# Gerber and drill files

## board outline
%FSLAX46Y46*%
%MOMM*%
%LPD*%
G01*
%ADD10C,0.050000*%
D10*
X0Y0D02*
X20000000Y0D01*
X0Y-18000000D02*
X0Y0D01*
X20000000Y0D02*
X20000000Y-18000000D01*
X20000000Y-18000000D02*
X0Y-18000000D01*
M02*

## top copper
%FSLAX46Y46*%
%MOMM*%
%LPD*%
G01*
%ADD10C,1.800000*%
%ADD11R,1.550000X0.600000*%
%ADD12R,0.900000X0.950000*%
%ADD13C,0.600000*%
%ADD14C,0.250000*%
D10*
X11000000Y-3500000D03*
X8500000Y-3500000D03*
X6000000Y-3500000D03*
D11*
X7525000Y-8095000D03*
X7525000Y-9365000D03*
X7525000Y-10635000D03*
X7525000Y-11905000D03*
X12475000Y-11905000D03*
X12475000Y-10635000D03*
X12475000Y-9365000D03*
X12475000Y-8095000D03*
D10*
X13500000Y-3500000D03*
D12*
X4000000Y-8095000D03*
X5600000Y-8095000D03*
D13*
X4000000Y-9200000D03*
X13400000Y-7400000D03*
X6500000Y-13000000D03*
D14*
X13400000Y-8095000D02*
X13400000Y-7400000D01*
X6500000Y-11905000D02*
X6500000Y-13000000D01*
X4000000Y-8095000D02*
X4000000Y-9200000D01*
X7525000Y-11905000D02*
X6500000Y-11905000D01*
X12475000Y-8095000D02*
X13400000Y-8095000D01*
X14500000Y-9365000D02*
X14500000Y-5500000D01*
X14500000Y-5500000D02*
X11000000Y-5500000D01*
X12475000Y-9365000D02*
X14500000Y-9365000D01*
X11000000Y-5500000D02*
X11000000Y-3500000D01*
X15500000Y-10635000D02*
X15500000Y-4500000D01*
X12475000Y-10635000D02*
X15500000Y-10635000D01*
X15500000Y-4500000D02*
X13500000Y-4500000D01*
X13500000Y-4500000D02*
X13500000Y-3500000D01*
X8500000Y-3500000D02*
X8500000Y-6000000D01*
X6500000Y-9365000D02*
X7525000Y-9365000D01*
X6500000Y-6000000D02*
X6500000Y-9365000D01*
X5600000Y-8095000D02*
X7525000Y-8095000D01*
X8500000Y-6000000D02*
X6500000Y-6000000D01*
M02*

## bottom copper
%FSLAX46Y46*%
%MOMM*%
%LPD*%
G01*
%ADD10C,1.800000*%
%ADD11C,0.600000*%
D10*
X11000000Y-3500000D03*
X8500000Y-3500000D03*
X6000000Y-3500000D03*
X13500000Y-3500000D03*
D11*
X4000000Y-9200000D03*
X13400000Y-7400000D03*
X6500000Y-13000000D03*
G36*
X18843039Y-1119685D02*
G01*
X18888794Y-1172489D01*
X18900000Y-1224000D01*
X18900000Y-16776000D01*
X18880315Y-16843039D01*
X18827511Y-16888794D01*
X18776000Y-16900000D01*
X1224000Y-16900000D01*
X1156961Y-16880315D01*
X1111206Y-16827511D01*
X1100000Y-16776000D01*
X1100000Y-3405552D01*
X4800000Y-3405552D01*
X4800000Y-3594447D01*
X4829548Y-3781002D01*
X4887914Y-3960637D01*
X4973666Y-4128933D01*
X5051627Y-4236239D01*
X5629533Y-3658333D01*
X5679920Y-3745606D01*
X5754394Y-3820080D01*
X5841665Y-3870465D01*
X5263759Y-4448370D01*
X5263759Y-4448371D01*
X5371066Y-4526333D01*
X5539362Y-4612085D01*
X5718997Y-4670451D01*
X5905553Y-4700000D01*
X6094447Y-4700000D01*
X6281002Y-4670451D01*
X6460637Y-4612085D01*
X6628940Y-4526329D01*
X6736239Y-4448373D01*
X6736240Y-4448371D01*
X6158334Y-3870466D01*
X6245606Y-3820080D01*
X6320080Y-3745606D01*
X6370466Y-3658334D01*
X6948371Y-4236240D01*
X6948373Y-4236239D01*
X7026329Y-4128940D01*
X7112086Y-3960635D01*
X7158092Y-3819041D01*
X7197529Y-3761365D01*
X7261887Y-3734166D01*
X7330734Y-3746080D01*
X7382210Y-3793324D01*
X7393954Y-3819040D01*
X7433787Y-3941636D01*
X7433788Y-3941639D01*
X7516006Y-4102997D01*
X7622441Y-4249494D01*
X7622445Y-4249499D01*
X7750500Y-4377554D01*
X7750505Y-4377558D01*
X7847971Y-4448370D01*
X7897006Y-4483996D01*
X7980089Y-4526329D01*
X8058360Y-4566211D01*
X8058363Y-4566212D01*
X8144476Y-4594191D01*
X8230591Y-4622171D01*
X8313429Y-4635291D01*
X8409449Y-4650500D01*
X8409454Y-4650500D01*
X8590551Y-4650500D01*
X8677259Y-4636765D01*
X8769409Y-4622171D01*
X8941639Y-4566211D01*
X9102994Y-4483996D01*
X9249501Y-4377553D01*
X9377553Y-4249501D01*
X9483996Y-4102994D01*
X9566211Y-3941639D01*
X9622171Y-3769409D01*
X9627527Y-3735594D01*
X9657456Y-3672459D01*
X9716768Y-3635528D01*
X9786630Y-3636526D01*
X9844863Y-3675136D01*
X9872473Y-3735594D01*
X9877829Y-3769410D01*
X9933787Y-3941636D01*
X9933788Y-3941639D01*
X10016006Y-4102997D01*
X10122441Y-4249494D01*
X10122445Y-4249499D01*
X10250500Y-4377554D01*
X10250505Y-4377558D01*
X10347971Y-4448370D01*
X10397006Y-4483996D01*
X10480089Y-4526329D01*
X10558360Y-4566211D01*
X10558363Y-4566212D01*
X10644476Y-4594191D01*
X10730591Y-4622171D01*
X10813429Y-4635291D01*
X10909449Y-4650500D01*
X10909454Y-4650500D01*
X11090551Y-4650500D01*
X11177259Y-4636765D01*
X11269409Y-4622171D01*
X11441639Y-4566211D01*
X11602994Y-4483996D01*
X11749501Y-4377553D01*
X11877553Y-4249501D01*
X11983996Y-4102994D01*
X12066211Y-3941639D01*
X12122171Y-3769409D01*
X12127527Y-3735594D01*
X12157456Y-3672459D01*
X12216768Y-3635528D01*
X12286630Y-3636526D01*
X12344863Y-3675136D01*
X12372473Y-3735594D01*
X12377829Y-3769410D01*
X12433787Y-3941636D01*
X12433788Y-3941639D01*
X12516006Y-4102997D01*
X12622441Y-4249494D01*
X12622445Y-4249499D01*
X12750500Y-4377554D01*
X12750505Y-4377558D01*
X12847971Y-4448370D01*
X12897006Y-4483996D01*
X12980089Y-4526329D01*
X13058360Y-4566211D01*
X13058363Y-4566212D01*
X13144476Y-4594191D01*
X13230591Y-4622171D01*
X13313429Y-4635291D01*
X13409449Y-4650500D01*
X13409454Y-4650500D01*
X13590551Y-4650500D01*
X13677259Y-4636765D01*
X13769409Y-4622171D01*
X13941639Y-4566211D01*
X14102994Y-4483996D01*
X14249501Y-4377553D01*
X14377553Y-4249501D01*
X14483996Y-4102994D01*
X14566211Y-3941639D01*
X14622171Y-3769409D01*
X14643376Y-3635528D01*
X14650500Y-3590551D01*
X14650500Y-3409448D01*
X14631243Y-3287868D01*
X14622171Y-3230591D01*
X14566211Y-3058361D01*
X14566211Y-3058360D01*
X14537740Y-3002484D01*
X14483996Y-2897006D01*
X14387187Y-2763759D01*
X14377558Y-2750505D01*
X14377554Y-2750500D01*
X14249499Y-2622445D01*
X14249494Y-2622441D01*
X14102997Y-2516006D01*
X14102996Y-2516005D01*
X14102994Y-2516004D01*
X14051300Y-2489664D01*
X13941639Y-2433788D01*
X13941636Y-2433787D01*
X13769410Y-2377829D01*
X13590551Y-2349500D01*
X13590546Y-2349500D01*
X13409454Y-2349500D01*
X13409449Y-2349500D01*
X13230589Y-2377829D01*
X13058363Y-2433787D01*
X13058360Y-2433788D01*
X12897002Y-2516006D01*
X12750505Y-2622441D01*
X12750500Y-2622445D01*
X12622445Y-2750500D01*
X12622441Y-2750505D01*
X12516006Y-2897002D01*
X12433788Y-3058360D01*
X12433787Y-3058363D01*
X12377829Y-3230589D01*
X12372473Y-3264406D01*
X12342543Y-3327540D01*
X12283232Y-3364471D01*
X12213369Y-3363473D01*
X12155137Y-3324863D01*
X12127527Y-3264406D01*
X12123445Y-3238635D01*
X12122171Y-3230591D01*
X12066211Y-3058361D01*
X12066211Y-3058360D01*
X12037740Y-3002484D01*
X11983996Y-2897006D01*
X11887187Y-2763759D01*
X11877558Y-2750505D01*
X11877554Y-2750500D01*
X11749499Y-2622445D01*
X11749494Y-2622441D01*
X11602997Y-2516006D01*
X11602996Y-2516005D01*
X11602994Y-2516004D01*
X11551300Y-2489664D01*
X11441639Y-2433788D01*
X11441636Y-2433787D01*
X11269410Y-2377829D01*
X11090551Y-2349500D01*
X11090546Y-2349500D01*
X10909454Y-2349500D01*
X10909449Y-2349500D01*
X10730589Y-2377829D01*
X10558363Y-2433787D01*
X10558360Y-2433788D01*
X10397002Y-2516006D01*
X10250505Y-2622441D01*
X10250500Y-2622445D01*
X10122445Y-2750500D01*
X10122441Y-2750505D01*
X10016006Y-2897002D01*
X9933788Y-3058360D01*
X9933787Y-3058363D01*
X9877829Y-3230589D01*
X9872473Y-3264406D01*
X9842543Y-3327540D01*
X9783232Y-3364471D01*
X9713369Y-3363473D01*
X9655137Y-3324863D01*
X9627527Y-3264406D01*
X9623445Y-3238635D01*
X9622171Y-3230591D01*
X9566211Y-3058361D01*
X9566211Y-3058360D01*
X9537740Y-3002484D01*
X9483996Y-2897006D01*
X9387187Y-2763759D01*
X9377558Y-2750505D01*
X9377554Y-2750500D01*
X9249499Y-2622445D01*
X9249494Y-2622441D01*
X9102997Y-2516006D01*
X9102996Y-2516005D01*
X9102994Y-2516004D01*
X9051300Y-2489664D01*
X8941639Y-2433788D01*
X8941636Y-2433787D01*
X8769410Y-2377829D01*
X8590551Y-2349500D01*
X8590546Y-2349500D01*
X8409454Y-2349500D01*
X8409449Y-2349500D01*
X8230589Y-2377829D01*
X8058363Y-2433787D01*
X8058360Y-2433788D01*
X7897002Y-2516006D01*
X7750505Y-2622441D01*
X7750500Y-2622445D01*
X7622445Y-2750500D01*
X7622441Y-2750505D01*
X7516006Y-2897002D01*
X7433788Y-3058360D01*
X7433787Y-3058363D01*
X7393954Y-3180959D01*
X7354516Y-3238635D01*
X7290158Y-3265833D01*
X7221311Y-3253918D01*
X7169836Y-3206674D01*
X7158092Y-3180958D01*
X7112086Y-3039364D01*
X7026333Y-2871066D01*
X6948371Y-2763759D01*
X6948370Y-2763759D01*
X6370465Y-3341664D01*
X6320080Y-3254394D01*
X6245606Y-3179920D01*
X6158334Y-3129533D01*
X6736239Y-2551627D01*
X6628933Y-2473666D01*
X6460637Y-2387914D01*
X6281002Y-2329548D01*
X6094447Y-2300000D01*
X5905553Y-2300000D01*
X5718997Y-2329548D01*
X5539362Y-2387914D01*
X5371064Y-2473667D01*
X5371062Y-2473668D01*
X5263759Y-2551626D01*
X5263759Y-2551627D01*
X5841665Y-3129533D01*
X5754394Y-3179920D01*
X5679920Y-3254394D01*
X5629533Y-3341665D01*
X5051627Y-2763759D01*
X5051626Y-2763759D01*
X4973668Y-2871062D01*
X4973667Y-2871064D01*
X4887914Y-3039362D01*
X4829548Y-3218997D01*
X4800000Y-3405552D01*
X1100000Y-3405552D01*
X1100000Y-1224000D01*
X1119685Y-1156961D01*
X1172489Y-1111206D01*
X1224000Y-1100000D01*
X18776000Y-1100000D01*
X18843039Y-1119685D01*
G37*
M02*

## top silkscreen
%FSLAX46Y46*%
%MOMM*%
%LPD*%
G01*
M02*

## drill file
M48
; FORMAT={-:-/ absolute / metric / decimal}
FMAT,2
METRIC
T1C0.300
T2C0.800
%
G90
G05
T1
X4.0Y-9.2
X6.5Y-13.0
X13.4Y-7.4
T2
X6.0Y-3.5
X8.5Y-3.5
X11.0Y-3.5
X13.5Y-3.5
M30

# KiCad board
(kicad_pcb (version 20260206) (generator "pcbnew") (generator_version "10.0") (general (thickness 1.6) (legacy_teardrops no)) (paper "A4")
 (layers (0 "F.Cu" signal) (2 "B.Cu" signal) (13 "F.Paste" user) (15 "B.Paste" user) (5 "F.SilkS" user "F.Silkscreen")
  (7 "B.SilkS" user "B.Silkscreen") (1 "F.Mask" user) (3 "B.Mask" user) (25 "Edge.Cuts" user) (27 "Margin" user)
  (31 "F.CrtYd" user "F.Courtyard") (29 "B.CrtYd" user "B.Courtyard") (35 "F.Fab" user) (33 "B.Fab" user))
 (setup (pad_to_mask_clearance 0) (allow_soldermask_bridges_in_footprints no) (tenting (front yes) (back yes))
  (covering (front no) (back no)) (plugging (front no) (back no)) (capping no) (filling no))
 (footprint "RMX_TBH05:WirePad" (layer "F.Cu") (at 11 3.5)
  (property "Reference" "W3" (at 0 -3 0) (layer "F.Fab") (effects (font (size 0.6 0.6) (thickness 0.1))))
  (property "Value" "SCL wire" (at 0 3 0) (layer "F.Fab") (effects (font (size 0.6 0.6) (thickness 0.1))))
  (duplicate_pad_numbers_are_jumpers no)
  (pad "1" thru_hole circle (at 0 0) (size 1.8 1.8) (drill 0.8) (layers "*.Cu" "*.Mask") (remove_unused_layers no) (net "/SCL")))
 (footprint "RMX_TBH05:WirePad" (layer "F.Cu") (at 8.5 3.5)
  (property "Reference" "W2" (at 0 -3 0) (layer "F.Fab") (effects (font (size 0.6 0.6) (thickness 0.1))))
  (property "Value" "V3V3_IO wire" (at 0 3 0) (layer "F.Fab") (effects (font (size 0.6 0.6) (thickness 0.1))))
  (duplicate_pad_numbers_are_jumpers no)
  (pad "1" thru_hole circle (at 0 0) (size 1.8 1.8) (drill 0.8) (layers "*.Cu" "*.Mask") (remove_unused_layers no) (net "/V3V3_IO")))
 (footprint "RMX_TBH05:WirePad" (layer "F.Cu") (at 6 3.5)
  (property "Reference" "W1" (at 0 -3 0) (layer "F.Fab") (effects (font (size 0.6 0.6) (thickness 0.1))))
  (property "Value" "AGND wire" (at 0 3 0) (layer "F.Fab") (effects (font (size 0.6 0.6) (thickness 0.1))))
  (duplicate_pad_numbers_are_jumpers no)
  (pad "1" thru_hole circle (at 0 0) (size 1.8 1.8) (drill 0.8) (layers "*.Cu" "*.Mask") (remove_unused_layers no) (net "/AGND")))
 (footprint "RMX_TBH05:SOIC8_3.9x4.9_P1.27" (layer "F.Cu") (at 10 10)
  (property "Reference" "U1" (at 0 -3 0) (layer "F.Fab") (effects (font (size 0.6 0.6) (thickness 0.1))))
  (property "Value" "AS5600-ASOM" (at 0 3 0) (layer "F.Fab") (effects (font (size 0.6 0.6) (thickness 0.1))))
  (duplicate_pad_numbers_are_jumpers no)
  (pad "1" smd rect (at -2.475 -1.905) (size 1.55 0.6) (layers "F.Cu" "F.Mask" "F.Paste") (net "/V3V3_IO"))
  (pad "2" smd rect (at -2.475 -0.635) (size 1.55 0.6) (layers "F.Cu" "F.Mask" "F.Paste") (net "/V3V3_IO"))
  (pad "3" smd rect (at -2.475 0.635) (size 1.55 0.6) (layers "F.Cu" "F.Mask" "F.Paste") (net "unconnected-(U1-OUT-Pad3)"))
  (pad "4" smd rect (at -2.475 1.905) (size 1.55 0.6) (layers "F.Cu" "F.Mask" "F.Paste") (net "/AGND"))
  (pad "5" smd rect (at 2.475 1.905) (size 1.55 0.6) (layers "F.Cu" "F.Mask" "F.Paste") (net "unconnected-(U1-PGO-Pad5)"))
  (pad "6" smd rect (at 2.475 0.635) (size 1.55 0.6) (layers "F.Cu" "F.Mask" "F.Paste") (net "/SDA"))
  (pad "7" smd rect (at 2.475 -0.635) (size 1.55 0.6) (layers "F.Cu" "F.Mask" "F.Paste") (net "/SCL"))
  (pad "8" smd rect (at 2.475 -1.905) (size 1.55 0.6) (layers "F.Cu" "F.Mask" "F.Paste") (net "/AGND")))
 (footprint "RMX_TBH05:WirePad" (layer "F.Cu") (at 13.5 3.5)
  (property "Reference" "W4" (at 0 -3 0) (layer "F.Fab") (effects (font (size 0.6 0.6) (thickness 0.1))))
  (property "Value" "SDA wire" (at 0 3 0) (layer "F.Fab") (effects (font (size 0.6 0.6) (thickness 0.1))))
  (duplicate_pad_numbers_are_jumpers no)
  (pad "1" thru_hole circle (at 0 0) (size 1.8 1.8) (drill 0.8) (layers "*.Cu" "*.Mask") (remove_unused_layers no) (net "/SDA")))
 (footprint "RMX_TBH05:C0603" (layer "F.Cu") (at 4.8 8.095)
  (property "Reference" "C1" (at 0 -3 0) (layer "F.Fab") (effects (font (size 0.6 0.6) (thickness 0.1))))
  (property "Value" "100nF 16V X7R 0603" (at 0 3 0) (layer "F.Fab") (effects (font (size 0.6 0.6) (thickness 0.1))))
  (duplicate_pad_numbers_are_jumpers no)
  (pad "1" smd rect (at -0.8 0) (size 0.9 0.95) (layers "F.Cu" "F.Mask" "F.Paste") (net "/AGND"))
  (pad "2" smd rect (at 0.8 0) (size 0.9 0.95) (layers "F.Cu" "F.Mask" "F.Paste") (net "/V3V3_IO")))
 (gr_line (start 0 0) (end 20 0) (stroke (width 0.05) (type default)) (layer "Edge.Cuts"))
 (gr_line (start 0 18) (end 0 0) (stroke (width 0.05) (type default)) (layer "Edge.Cuts"))
 (gr_line (start 20 0) (end 20 18) (stroke (width 0.05) (type default)) (layer "Edge.Cuts"))
 (gr_line (start 20 18) (end 0 18) (stroke (width 0.05) (type default)) (layer "Edge.Cuts"))
 (segment (start 13.4 8.095) (end 13.4 7.4) (width 0.25) (layer "F.Cu") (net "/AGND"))
 (segment (start 6.5 11.905) (end 6.5 13) (width 0.25) (layer "F.Cu") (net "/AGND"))
 (segment (start 4 8.095) (end 4 9.2) (width 0.25) (layer "F.Cu") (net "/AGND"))
 (segment (start 7.525 11.905) (end 6.5 11.905) (width 0.25) (layer "F.Cu") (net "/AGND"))
 (segment (start 12.475 8.095) (end 13.4 8.095) (width 0.25) (layer "F.Cu") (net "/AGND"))
 (via (at 4 9.2) (size 0.6) (drill 0.3) (layers "F.Cu" "B.Cu") (capping no) (covering (front no) (back no)) (plugging (front no) (back no))
  (filling no) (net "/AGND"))
 (via (at 13.4 7.4) (size 0.6) (drill 0.3) (layers "F.Cu" "B.Cu") (capping no) (covering (front no) (back no))
  (plugging (front no) (back no)) (filling no) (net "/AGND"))
 (via (at 6.5 13) (size 0.6) (drill 0.3) (layers "F.Cu" "B.Cu") (capping no) (covering (front no) (back no)) (plugging (front no) (back no))
  (filling no) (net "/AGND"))
 (segment (start 14.5 9.365) (end 14.5 5.5) (width 0.25) (layer "F.Cu") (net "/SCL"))
 (segment (start 14.5 5.5) (end 11 5.5) (width 0.25) (layer "F.Cu") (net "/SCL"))
 (segment (start 12.475 9.365) (end 14.5 9.365) (width 0.25) (layer "F.Cu") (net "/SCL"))
 (segment (start 11 5.5) (end 11 3.5) (width 0.25) (layer "F.Cu") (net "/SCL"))
 (segment (start 15.5 10.635) (end 15.5 4.5) (width 0.25) (layer "F.Cu") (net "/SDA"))
 (segment (start 12.475 10.635) (end 15.5 10.635) (width 0.25) (layer "F.Cu") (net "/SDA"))
 (segment (start 15.5 4.5) (end 13.5 4.5) (width 0.25) (layer "F.Cu") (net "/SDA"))
 (segment (start 13.5 4.5) (end 13.5 3.5) (width 0.25) (layer "F.Cu") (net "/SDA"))
 (segment (start 8.5 3.5) (end 8.5 6) (width 0.25) (layer "F.Cu") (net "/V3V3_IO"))
 (segment (start 6.5 9.365) (end 7.525 9.365) (width 0.25) (layer "F.Cu") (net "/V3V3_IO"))
 (segment (start 6.5 6) (end 6.5 9.365) (width 0.25) (layer "F.Cu") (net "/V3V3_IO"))
 (segment (start 5.6 8.095) (end 7.525 8.095) (width 0.25) (layer "F.Cu") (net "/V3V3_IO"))
 (segment (start 8.5 6) (end 6.5 6) (width 0.25) (layer "F.Cu") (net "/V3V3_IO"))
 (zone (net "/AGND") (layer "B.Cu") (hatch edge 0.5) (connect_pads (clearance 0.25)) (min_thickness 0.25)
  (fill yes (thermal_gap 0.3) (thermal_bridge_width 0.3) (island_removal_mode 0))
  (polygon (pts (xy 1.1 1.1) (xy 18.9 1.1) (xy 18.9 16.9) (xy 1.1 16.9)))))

